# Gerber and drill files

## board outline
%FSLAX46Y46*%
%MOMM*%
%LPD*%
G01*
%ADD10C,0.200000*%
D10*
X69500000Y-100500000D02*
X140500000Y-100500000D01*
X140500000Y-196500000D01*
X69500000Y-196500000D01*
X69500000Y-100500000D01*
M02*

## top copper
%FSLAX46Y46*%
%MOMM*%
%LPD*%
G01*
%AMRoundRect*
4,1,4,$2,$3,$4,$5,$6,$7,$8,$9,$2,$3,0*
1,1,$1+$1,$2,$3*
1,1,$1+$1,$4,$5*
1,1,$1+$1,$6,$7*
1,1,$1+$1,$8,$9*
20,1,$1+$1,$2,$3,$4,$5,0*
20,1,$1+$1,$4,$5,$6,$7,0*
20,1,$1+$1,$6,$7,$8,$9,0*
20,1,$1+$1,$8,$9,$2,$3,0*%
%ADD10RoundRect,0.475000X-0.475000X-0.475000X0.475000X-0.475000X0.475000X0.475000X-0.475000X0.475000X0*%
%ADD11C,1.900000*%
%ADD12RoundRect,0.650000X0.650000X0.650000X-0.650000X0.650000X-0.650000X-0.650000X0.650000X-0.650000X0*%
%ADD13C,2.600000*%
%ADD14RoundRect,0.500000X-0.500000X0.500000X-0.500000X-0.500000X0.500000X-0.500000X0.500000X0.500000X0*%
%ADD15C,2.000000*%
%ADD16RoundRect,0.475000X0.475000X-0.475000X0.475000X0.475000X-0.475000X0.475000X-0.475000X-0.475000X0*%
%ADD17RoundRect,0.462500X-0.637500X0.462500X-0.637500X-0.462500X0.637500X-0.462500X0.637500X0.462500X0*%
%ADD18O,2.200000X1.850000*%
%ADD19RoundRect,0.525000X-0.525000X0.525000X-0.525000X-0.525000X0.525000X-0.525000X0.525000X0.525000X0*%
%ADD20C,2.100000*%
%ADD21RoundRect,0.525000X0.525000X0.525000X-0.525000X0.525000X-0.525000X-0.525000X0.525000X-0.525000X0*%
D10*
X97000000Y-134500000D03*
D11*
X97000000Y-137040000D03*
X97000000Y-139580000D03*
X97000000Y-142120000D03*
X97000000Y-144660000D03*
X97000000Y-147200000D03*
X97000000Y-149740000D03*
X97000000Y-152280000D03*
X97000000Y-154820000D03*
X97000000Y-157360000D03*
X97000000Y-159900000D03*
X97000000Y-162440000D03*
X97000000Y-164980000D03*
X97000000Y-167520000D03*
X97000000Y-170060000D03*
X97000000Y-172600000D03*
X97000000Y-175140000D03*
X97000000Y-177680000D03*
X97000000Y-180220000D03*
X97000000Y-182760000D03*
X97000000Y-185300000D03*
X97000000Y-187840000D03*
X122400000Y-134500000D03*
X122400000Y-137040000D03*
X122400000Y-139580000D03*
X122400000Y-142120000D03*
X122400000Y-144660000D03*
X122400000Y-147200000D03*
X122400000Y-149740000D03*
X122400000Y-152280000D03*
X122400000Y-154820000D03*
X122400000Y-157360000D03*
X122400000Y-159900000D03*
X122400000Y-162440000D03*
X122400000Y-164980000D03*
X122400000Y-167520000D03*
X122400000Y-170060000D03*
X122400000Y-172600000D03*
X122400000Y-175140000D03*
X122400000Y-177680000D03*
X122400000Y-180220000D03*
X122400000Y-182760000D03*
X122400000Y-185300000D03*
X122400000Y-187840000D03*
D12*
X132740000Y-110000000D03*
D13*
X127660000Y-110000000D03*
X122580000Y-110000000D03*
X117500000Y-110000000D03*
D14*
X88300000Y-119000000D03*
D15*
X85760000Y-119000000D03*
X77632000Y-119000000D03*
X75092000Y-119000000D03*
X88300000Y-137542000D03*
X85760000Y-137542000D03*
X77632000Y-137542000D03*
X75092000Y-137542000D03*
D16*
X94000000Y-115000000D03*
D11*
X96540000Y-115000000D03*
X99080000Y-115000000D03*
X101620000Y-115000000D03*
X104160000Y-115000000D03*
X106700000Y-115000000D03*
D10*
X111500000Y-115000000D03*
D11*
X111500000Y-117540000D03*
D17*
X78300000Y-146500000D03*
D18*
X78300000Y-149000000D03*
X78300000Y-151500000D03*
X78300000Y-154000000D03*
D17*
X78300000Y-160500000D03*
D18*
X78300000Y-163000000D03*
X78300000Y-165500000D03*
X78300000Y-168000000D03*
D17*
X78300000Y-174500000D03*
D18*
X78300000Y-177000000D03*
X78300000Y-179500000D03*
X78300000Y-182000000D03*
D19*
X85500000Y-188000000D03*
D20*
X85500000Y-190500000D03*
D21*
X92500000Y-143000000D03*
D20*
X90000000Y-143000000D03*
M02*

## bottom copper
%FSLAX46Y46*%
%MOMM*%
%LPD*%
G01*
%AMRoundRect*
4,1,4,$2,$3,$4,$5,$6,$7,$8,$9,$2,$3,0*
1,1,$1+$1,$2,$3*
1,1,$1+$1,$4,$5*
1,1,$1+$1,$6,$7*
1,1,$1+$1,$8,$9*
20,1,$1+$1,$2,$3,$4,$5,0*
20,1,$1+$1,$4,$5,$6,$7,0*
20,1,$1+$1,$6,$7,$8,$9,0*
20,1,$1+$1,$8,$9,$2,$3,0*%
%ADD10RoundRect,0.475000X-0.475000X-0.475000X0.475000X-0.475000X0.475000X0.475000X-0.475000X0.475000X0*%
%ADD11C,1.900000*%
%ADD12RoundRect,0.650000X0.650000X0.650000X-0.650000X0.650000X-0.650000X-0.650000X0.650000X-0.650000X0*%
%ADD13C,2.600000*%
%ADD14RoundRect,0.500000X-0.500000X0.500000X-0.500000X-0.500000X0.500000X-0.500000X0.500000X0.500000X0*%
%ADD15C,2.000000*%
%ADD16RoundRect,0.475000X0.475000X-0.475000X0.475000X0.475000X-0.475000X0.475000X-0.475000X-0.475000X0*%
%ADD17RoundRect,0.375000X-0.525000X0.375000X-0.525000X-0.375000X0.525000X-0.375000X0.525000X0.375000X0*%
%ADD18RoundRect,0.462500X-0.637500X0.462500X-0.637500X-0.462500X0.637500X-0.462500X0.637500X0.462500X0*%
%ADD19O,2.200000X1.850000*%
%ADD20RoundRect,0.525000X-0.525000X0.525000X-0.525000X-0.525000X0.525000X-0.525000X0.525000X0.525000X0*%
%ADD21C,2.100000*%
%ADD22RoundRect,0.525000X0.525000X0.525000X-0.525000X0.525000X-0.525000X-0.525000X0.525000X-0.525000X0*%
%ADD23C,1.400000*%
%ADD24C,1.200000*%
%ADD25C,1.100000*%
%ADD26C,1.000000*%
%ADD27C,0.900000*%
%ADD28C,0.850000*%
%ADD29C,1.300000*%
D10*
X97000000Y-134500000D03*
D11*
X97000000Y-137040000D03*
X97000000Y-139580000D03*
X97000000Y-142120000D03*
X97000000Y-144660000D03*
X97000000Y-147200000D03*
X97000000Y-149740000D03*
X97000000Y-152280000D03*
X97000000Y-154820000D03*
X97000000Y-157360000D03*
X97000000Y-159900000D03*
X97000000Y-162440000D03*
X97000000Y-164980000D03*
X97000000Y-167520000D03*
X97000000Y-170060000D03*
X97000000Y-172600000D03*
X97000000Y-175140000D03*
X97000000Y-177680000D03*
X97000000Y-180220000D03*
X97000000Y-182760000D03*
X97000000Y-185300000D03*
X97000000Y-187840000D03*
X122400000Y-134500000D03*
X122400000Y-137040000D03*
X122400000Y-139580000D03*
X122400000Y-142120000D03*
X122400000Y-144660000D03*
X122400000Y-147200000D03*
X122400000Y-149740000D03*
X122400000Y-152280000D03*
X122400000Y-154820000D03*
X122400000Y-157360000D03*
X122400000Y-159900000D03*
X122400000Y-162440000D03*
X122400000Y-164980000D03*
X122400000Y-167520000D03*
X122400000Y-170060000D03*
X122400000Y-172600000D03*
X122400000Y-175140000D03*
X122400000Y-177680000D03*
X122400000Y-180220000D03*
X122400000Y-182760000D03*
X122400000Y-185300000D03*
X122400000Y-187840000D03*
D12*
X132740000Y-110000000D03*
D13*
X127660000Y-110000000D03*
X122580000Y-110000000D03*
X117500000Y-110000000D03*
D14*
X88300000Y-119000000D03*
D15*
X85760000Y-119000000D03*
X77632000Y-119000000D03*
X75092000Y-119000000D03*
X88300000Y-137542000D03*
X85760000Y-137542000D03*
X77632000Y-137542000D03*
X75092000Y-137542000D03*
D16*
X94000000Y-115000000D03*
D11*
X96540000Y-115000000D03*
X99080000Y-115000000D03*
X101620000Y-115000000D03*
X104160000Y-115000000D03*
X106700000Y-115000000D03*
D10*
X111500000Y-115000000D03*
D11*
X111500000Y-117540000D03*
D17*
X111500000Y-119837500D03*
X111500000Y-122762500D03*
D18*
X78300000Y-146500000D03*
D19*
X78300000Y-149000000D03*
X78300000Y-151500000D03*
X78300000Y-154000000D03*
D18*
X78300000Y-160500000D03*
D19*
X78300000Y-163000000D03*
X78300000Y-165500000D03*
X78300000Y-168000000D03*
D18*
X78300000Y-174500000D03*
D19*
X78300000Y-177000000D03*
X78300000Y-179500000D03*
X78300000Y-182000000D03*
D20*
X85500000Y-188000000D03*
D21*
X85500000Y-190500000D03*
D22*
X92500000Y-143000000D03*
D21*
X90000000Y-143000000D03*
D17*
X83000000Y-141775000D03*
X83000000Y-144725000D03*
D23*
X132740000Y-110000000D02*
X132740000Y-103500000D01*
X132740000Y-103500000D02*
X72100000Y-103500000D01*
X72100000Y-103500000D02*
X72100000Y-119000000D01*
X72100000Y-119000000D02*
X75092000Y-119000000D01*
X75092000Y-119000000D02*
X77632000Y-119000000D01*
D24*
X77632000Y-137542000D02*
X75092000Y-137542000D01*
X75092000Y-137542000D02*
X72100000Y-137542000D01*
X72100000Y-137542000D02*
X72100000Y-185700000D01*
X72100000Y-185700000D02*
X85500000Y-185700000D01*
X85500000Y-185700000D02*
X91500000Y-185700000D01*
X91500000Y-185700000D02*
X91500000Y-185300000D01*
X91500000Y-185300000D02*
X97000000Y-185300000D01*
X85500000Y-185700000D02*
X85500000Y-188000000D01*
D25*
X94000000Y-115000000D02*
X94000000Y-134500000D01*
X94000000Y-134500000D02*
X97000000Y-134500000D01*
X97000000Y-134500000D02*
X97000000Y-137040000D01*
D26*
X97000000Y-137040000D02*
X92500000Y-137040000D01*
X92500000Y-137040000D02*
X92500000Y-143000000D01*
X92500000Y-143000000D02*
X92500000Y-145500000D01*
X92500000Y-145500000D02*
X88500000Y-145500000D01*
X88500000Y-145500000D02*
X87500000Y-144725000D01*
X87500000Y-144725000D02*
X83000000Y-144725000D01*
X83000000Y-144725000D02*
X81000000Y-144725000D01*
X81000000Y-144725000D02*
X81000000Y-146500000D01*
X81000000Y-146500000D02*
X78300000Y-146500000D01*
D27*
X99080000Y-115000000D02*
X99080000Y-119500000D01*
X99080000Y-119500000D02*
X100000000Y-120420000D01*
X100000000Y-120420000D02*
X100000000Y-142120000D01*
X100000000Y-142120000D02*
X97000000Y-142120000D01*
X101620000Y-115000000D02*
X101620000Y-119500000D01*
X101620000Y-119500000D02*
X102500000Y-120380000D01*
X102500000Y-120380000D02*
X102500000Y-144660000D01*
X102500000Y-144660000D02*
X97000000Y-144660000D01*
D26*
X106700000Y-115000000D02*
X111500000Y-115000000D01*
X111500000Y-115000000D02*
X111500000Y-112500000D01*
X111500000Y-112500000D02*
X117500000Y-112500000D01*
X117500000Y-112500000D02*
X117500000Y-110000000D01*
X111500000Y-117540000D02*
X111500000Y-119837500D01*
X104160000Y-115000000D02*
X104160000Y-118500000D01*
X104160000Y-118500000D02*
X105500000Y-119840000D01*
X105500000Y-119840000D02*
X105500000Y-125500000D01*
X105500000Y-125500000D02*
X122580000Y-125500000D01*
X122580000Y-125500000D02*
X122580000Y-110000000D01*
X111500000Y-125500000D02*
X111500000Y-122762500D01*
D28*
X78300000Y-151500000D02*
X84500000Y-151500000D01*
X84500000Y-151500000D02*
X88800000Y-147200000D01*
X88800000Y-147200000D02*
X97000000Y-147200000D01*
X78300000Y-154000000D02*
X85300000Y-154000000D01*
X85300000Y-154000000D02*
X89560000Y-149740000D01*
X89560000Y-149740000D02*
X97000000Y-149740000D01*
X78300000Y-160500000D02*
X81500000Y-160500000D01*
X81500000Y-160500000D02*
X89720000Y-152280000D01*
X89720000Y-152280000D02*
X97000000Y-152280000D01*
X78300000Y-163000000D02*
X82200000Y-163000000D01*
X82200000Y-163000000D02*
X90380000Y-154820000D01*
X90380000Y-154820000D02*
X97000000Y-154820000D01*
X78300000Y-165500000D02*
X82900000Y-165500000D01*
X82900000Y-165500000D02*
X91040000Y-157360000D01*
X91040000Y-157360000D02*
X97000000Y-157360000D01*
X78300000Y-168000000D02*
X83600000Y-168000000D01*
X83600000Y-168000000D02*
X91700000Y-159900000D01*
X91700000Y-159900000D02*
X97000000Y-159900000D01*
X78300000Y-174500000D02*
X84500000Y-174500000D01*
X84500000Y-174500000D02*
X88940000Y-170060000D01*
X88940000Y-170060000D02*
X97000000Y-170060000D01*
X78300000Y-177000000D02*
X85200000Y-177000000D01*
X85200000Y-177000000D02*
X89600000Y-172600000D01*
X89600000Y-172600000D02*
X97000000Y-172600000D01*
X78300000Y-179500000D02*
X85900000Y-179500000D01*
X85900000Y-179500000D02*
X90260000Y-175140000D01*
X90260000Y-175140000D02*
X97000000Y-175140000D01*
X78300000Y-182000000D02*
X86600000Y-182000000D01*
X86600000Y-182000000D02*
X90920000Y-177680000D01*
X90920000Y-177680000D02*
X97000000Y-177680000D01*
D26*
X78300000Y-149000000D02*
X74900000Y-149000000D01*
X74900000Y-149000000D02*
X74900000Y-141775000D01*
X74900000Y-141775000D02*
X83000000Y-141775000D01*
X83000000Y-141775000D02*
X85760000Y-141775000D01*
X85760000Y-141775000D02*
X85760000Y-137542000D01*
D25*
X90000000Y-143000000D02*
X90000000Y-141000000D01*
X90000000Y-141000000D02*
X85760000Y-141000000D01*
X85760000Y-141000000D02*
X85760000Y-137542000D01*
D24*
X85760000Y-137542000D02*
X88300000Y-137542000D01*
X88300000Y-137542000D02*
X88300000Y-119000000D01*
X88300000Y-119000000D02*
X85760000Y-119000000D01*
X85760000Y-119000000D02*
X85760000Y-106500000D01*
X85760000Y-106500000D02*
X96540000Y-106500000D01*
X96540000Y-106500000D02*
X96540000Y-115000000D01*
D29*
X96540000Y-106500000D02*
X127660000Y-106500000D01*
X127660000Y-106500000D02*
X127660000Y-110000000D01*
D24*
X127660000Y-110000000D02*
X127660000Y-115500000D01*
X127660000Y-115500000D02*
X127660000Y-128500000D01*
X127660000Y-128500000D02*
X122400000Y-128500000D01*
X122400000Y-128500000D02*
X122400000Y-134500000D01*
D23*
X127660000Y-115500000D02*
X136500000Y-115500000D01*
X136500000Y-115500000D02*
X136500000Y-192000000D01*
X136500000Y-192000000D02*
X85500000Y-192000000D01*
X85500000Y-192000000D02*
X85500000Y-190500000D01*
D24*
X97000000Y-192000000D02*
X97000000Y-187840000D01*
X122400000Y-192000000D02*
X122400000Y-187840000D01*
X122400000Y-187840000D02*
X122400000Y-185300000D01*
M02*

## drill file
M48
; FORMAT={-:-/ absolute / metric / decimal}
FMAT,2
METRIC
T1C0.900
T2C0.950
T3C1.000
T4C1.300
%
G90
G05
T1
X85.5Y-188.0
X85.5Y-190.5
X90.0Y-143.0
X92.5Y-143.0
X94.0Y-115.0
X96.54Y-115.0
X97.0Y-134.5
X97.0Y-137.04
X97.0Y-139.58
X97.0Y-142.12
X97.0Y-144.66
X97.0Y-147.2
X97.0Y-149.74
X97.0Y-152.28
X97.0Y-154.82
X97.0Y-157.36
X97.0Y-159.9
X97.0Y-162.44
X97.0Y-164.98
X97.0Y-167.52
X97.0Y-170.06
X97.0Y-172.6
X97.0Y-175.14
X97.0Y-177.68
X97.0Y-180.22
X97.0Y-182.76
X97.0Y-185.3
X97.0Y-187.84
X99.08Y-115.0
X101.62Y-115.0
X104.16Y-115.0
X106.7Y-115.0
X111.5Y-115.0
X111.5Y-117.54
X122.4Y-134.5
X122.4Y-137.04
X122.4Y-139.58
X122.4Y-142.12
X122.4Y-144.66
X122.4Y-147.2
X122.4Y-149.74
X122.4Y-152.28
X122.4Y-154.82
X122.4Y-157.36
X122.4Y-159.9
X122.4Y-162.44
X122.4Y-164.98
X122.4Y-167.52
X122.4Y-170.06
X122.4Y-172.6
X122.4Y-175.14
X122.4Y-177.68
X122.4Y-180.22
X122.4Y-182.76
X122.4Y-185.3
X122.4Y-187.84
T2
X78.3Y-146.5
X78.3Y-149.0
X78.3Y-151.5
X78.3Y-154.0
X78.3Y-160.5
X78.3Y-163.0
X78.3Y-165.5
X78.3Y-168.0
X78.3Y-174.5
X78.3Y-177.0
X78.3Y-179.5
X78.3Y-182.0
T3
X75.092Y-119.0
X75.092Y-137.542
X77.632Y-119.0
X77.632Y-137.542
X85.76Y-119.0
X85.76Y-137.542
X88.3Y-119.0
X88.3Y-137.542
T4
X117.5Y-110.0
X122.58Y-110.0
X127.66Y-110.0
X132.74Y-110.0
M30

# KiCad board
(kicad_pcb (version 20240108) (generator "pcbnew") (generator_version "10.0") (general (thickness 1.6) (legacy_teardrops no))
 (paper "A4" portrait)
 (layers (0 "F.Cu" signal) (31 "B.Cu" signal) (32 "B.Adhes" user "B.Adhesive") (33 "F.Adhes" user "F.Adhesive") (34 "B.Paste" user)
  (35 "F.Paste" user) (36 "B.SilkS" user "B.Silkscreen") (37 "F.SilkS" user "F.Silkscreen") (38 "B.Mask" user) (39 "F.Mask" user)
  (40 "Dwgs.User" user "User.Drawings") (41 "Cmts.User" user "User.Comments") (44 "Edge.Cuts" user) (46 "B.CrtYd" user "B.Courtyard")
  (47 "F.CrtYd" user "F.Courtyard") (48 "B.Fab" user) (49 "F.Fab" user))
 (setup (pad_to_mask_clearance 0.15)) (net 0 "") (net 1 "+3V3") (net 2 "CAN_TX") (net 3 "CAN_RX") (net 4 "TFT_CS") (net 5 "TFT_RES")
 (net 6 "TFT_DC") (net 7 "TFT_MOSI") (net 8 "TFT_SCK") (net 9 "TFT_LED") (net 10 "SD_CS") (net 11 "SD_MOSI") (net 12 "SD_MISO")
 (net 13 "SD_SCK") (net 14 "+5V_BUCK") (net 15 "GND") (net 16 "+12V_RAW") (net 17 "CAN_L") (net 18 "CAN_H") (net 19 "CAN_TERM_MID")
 (gr_rect (start 69.500 100.500) (end 140.500 196.500) (stroke (width 0.2) (type default)) (fill none) (layer "Edge.Cuts"))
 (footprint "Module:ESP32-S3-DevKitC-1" (layer "F.Cu") (at 97.0000 134.5000 0)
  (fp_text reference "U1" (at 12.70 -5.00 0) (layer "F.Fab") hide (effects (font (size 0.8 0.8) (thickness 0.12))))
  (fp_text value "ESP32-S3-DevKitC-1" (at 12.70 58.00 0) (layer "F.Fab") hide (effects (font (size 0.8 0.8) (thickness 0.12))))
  (pad "L1" thru_hole roundrect (at 0.0000 0.0000 0) (size 1.90 1.90) (drill 0.90) (layers "*.Cu" "*.Mask") (roundrect_rratio 0.25)
   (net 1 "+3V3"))
  (pad "L2" thru_hole circle (at 0.0000 2.5400 0) (size 1.90 1.90) (drill 0.90) (layers "*.Cu" "*.Mask") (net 1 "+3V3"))
  (pad "L3" thru_hole circle (at 0.0000 5.0800 0) (size 1.90 1.90) (drill 0.90) (layers "*.Cu" "*.Mask"))
  (pad "L4" thru_hole circle (at 0.0000 7.6200 0) (size 1.90 1.90) (drill 0.90) (layers "*.Cu" "*.Mask") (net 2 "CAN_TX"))
  (pad "L5" thru_hole circle (at 0.0000 10.1600 0) (size 1.90 1.90) (drill 0.90) (layers "*.Cu" "*.Mask") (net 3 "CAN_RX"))
  (pad "L6" thru_hole circle (at 0.0000 12.7000 0) (size 1.90 1.90) (drill 0.90) (layers "*.Cu" "*.Mask") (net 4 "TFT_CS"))
  (pad "L7" thru_hole circle (at 0.0000 15.2400 0) (size 1.90 1.90) (drill 0.90) (layers "*.Cu" "*.Mask") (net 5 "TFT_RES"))
  (pad "L8" thru_hole circle (at 0.0000 17.7800 0) (size 1.90 1.90) (drill 0.90) (layers "*.Cu" "*.Mask") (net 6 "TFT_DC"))
  (pad "L9" thru_hole circle (at 0.0000 20.3200 0) (size 1.90 1.90) (drill 0.90) (layers "*.Cu" "*.Mask") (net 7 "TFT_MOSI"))
  (pad "L10" thru_hole circle (at 0.0000 22.8600 0) (size 1.90 1.90) (drill 0.90) (layers "*.Cu" "*.Mask") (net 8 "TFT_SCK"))
  (pad "L11" thru_hole circle (at 0.0000 25.4000 0) (size 1.90 1.90) (drill 0.90) (layers "*.Cu" "*.Mask") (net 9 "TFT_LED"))
  (pad "L12" thru_hole circle (at 0.0000 27.9400 0) (size 1.90 1.90) (drill 0.90) (layers "*.Cu" "*.Mask"))
  (pad "L13" thru_hole circle (at 0.0000 30.4800 0) (size 1.90 1.90) (drill 0.90) (layers "*.Cu" "*.Mask"))
  (pad "L14" thru_hole circle (at 0.0000 33.0200 0) (size 1.90 1.90) (drill 0.90) (layers "*.Cu" "*.Mask"))
  (pad "L15" thru_hole circle (at 0.0000 35.5600 0) (size 1.90 1.90) (drill 0.90) (layers "*.Cu" "*.Mask") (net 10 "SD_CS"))
  (pad "L16" thru_hole circle (at 0.0000 38.1000 0) (size 1.90 1.90) (drill 0.90) (layers "*.Cu" "*.Mask") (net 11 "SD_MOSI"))
  (pad "L17" thru_hole circle (at 0.0000 40.6400 0) (size 1.90 1.90) (drill 0.90) (layers "*.Cu" "*.Mask") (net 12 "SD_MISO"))
  (pad "L18" thru_hole circle (at 0.0000 43.1800 0) (size 1.90 1.90) (drill 0.90) (layers "*.Cu" "*.Mask") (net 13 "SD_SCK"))
  (pad "L19" thru_hole circle (at 0.0000 45.7200 0) (size 1.90 1.90) (drill 0.90) (layers "*.Cu" "*.Mask"))
  (pad "L20" thru_hole circle (at 0.0000 48.2600 0) (size 1.90 1.90) (drill 0.90) (layers "*.Cu" "*.Mask"))
  (pad "L21" thru_hole circle (at 0.0000 50.8000 0) (size 1.90 1.90) (drill 0.90) (layers "*.Cu" "*.Mask") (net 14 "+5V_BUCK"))
  (pad "L22" thru_hole circle (at 0.0000 53.3400 0) (size 1.90 1.90) (drill 0.90) (layers "*.Cu" "*.Mask") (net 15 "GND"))
  (pad "R1" thru_hole circle (at 25.4000 0.0000 0) (size 1.90 1.90) (drill 0.90) (layers "*.Cu" "*.Mask") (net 15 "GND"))
  (pad "R2" thru_hole circle (at 25.4000 2.5400 0) (size 1.90 1.90) (drill 0.90) (layers "*.Cu" "*.Mask"))
  (pad "R3" thru_hole circle (at 25.4000 5.0800 0) (size 1.90 1.90) (drill 0.90) (layers "*.Cu" "*.Mask"))
  (pad "R4" thru_hole circle (at 25.4000 7.6200 0) (size 1.90 1.90) (drill 0.90) (layers "*.Cu" "*.Mask"))
  (pad "R5" thru_hole circle (at 25.4000 10.1600 0) (size 1.90 1.90) (drill 0.90) (layers "*.Cu" "*.Mask"))
  (pad "R6" thru_hole circle (at 25.4000 12.7000 0) (size 1.90 1.90) (drill 0.90) (layers "*.Cu" "*.Mask"))
  (pad "R7" thru_hole circle (at 25.4000 15.2400 0) (size 1.90 1.90) (drill 0.90) (layers "*.Cu" "*.Mask"))
  (pad "R8" thru_hole circle (at 25.4000 17.7800 0) (size 1.90 1.90) (drill 0.90) (layers "*.Cu" "*.Mask"))
  (pad "R9" thru_hole circle (at 25.4000 20.3200 0) (size 1.90 1.90) (drill 0.90) (layers "*.Cu" "*.Mask"))
  (pad "R10" thru_hole circle (at 25.4000 22.8600 0) (size 1.90 1.90) (drill 0.90) (layers "*.Cu" "*.Mask"))
  (pad "R11" thru_hole circle (at 25.4000 25.4000 0) (size 1.90 1.90) (drill 0.90) (layers "*.Cu" "*.Mask"))
  (pad "R12" thru_hole circle (at 25.4000 27.9400 0) (size 1.90 1.90) (drill 0.90) (layers "*.Cu" "*.Mask"))
  (pad "R13" thru_hole circle (at 25.4000 30.4800 0) (size 1.90 1.90) (drill 0.90) (layers "*.Cu" "*.Mask"))
  (pad "R14" thru_hole circle (at 25.4000 33.0200 0) (size 1.90 1.90) (drill 0.90) (layers "*.Cu" "*.Mask"))
  (pad "R15" thru_hole circle (at 25.4000 35.5600 0) (size 1.90 1.90) (drill 0.90) (layers "*.Cu" "*.Mask"))
  (pad "R16" thru_hole circle (at 25.4000 38.1000 0) (size 1.90 1.90) (drill 0.90) (layers "*.Cu" "*.Mask"))
  (pad "R17" thru_hole circle (at 25.4000 40.6400 0) (size 1.90 1.90) (drill 0.90) (layers "*.Cu" "*.Mask"))
  (pad "R18" thru_hole circle (at 25.4000 43.1800 0) (size 1.90 1.90) (drill 0.90) (layers "*.Cu" "*.Mask"))
  (pad "R19" thru_hole circle (at 25.4000 45.7200 0) (size 1.90 1.90) (drill 0.90) (layers "*.Cu" "*.Mask"))
  (pad "R20" thru_hole circle (at 25.4000 48.2600 0) (size 1.90 1.90) (drill 0.90) (layers "*.Cu" "*.Mask"))
  (pad "R21" thru_hole circle (at 25.4000 50.8000 0) (size 1.90 1.90) (drill 0.90) (layers "*.Cu" "*.Mask") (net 15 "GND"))
  (pad "R22" thru_hole circle (at 25.4000 53.3400 0) (size 1.90 1.90) (drill 0.90) (layers "*.Cu" "*.Mask") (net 15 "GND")))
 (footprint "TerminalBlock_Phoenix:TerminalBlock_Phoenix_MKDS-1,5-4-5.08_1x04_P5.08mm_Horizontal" (layer "F.Cu") (at 132.7400 110.0000 180)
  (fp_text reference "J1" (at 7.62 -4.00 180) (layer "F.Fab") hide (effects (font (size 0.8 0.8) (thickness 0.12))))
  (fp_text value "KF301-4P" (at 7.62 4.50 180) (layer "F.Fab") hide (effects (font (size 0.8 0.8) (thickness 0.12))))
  (pad "1" thru_hole roundrect (at 0.0000 0.0000 180) (size 2.60 2.60) (drill 1.30) (layers "*.Cu" "*.Mask") (roundrect_rratio 0.25)
   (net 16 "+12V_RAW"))
  (pad "2" thru_hole circle (at 5.0800 0.0000 180) (size 2.60 2.60) (drill 1.30) (layers "*.Cu" "*.Mask") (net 15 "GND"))
  (pad "3" thru_hole circle (at 10.1600 0.0000 180) (size 2.60 2.60) (drill 1.30) (layers "*.Cu" "*.Mask") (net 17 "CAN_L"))
  (pad "4" thru_hole circle (at 15.2400 0.0000 180) (size 2.60 2.60) (drill 1.30) (layers "*.Cu" "*.Mask") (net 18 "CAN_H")))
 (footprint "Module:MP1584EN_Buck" (layer "F.Cu") (at 88.3000 119.0000 270)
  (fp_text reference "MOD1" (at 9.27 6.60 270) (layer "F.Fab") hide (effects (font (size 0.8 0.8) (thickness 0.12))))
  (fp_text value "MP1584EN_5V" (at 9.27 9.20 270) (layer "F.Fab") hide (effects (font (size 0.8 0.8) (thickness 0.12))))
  (pad "1a" thru_hole roundrect (at 0.0000 0.0000 270) (size 2.00 2.00) (drill 1.00) (layers "*.Cu" "*.Mask") (roundrect_rratio 0.25)
   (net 15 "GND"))
  (pad "1b" thru_hole circle (at 0.0000 2.5400 270) (size 2.00 2.00) (drill 1.00) (layers "*.Cu" "*.Mask") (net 15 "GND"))
  (pad "2b" thru_hole circle (at 0.0000 10.6680 270) (size 2.00 2.00) (drill 1.00) (layers "*.Cu" "*.Mask") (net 16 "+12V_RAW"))
  (pad "2a" thru_hole circle (at 0.0000 13.2080 270) (size 2.00 2.00) (drill 1.00) (layers "*.Cu" "*.Mask") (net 16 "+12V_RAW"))
  (pad "3a" thru_hole circle (at 18.5420 0.0000 270) (size 2.00 2.00) (drill 1.00) (layers "*.Cu" "*.Mask") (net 15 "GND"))
  (pad "3b" thru_hole circle (at 18.5420 2.5400 270) (size 2.00 2.00) (drill 1.00) (layers "*.Cu" "*.Mask") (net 15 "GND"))
  (pad "4b" thru_hole circle (at 18.5420 10.6680 270) (size 2.00 2.00) (drill 1.00) (layers "*.Cu" "*.Mask") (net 14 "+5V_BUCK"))
  (pad "4a" thru_hole circle (at 18.5420 13.2080 270) (size 2.00 2.00) (drill 1.00) (layers "*.Cu" "*.Mask") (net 14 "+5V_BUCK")))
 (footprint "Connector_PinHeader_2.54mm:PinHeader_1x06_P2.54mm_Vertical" (layer "F.Cu") (at 94.0000 115.0000 90)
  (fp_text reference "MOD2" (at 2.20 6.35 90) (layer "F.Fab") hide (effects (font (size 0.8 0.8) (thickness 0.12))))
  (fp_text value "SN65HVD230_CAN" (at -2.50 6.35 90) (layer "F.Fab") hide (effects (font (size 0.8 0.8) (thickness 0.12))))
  (pad "1" thru_hole roundrect (at 0.0000 0.0000 90) (size 1.90 1.90) (drill 0.90) (layers "*.Cu" "*.Mask") (roundrect_rratio 0.25)
   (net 1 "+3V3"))
  (pad "2" thru_hole circle (at 0.0000 2.5400 90) (size 1.90 1.90) (drill 0.90) (layers "*.Cu" "*.Mask") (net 15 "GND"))
  (pad "3" thru_hole circle (at 0.0000 5.0800 90) (size 1.90 1.90) (drill 0.90) (layers "*.Cu" "*.Mask") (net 2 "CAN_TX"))
  (pad "4" thru_hole circle (at 0.0000 7.6200 90) (size 1.90 1.90) (drill 0.90) (layers "*.Cu" "*.Mask") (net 3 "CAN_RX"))
  (pad "5" thru_hole circle (at 0.0000 10.1600 90) (size 1.90 1.90) (drill 0.90) (layers "*.Cu" "*.Mask") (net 17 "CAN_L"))
  (pad "6" thru_hole circle (at 0.0000 12.7000 90) (size 1.90 1.90) (drill 0.90) (layers "*.Cu" "*.Mask") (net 18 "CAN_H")))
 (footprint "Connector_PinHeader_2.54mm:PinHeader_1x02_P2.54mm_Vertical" (layer "F.Cu") (at 111.5000 115.0000 0)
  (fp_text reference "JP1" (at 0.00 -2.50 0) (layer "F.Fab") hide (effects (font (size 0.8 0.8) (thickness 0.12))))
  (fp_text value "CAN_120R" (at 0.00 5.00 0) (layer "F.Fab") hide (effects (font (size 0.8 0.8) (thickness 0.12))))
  (pad "1" thru_hole roundrect (at 0.0000 0.0000 0) (size 1.90 1.90) (drill 0.90) (layers "*.Cu" "*.Mask") (roundrect_rratio 0.25)
   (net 18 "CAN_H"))
  (pad "2" thru_hole circle (at 0.0000 2.5400 0) (size 1.90 1.90) (drill 0.90) (layers "*.Cu" "*.Mask") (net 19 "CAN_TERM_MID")))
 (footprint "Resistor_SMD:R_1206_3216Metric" (layer "B.Cu") (at 111.5000 121.3000 270)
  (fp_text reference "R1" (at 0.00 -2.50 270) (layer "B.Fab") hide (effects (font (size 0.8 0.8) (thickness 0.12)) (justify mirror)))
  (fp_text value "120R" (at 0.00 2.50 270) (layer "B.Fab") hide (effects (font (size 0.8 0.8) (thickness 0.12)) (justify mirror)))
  (pad "1" smd roundrect (at -1.4625 0.0000 270) (size 1.50 1.80) (layers "B.Cu" "B.Mask" "B.Paste") (roundrect_rratio 0.25)
   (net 19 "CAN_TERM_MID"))
  (pad "2" smd roundrect (at 1.4625 0.0000 270) (size 1.50 1.80) (layers "B.Cu" "B.Mask" "B.Paste") (roundrect_rratio 0.25) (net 17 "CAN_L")))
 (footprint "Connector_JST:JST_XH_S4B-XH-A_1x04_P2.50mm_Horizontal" (layer "F.Cu") (at 78.3000 146.5000 270)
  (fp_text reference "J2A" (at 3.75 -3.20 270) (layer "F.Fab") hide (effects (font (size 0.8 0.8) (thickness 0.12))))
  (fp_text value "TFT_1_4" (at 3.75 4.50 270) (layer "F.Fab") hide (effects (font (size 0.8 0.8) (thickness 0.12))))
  (pad "1" thru_hole roundrect (at 0.0000 0.0000 270) (size 1.85 2.20) (drill 0.95) (layers "*.Cu" "*.Mask") (roundrect_rratio 0.25)
   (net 1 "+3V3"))
  (pad "2" thru_hole oval (at 2.5000 0.0000 270) (size 1.85 2.20) (drill 0.95) (layers "*.Cu" "*.Mask") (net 15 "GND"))
  (pad "3" thru_hole oval (at 5.0000 0.0000 270) (size 1.85 2.20) (drill 0.95) (layers "*.Cu" "*.Mask") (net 4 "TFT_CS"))
  (pad "4" thru_hole oval (at 7.5000 0.0000 270) (size 1.85 2.20) (drill 0.95) (layers "*.Cu" "*.Mask") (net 5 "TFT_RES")))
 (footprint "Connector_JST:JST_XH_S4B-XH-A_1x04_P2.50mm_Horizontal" (layer "F.Cu") (at 78.3000 160.5000 270)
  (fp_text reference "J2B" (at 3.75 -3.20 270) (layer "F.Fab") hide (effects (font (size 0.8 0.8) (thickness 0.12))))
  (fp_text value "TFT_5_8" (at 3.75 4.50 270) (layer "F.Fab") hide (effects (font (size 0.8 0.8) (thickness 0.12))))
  (pad "1" thru_hole roundrect (at 0.0000 0.0000 270) (size 1.85 2.20) (drill 0.95) (layers "*.Cu" "*.Mask") (roundrect_rratio 0.25)
   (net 6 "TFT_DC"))
  (pad "2" thru_hole oval (at 2.5000 0.0000 270) (size 1.85 2.20) (drill 0.95) (layers "*.Cu" "*.Mask") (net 7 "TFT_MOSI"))
  (pad "3" thru_hole oval (at 5.0000 0.0000 270) (size 1.85 2.20) (drill 0.95) (layers "*.Cu" "*.Mask") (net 8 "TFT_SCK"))
  (pad "4" thru_hole oval (at 7.5000 0.0000 270) (size 1.85 2.20) (drill 0.95) (layers "*.Cu" "*.Mask") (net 9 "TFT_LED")))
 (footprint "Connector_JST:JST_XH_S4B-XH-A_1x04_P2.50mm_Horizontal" (layer "F.Cu") (at 78.3000 174.5000 270)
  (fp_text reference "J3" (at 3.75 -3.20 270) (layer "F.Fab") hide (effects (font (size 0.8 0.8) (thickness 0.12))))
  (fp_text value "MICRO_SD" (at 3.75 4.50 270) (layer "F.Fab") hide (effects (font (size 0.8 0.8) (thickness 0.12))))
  (pad "1" thru_hole roundrect (at 0.0000 0.0000 270) (size 1.85 2.20) (drill 0.95) (layers "*.Cu" "*.Mask") (roundrect_rratio 0.25)
   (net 10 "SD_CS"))
  (pad "2" thru_hole oval (at 2.5000 0.0000 270) (size 1.85 2.20) (drill 0.95) (layers "*.Cu" "*.Mask") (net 11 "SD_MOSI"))
  (pad "3" thru_hole oval (at 5.0000 0.0000 270) (size 1.85 2.20) (drill 0.95) (layers "*.Cu" "*.Mask") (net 12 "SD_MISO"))
  (pad "4" thru_hole oval (at 7.5000 0.0000 270) (size 1.85 2.20) (drill 0.95) (layers "*.Cu" "*.Mask") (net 13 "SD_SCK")))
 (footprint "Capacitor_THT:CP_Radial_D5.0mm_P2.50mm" (layer "F.Cu") (at 85.5000 188.0000 270)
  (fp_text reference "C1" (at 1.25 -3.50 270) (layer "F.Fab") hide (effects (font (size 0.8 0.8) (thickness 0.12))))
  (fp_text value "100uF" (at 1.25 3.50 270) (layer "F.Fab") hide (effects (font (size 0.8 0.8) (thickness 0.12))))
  (pad "1" thru_hole roundrect (at 0.0000 0.0000 270) (size 2.10 2.10) (drill 0.90) (layers "*.Cu" "*.Mask") (roundrect_rratio 0.25)
   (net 14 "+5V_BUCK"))
  (pad "2" thru_hole circle (at 2.5000 0.0000 270) (size 2.10 2.10) (drill 0.90) (layers "*.Cu" "*.Mask") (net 15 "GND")))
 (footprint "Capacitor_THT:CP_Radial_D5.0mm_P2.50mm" (layer "F.Cu") (at 92.5000 143.0000 180)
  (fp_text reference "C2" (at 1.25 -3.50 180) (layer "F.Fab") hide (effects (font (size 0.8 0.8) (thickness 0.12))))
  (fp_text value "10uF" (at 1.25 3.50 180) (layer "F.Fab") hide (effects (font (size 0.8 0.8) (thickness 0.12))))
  (pad "1" thru_hole roundrect (at 0.0000 0.0000 180) (size 2.10 2.10) (drill 0.90) (layers "*.Cu" "*.Mask") (roundrect_rratio 0.25)
   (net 1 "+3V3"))
  (pad "2" thru_hole circle (at 2.5000 0.0000 180) (size 2.10 2.10) (drill 0.90) (layers "*.Cu" "*.Mask") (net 15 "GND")))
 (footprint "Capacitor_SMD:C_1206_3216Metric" (layer "B.Cu") (at 83.0000 143.2500 270)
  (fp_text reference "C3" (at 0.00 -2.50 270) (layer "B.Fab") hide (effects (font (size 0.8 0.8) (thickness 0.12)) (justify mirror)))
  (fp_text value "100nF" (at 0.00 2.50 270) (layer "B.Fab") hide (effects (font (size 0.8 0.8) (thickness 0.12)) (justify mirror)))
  (pad "1" smd roundrect (at -1.4750 0.0000 270) (size 1.50 1.80) (layers "B.Cu" "B.Mask" "B.Paste") (roundrect_rratio 0.25) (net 15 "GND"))
  (pad "2" smd roundrect (at 1.4750 0.0000 270) (size 1.50 1.80) (layers "B.Cu" "B.Mask" "B.Paste") (roundrect_rratio 0.25) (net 1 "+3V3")))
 (segment (start 132.7400 110.0000) (end 132.7400 103.5000) (width 1.40) (layer "B.Cu") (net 16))
 (segment (start 132.7400 103.5000) (end 72.1000 103.5000) (width 1.40) (layer "B.Cu") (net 16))
 (segment (start 72.1000 103.5000) (end 72.1000 119.0000) (width 1.40) (layer "B.Cu") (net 16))
 (segment (start 72.1000 119.0000) (end 75.0920 119.0000) (width 1.40) (layer "B.Cu") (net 16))
 (segment (start 75.0920 119.0000) (end 77.6320 119.0000) (width 1.40) (layer "B.Cu") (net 16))
 (segment (start 77.6320 137.5420) (end 75.0920 137.5420) (width 1.20) (layer "B.Cu") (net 14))
 (segment (start 75.0920 137.5420) (end 72.1000 137.5420) (width 1.20) (layer "B.Cu") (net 14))
 (segment (start 72.1000 137.5420) (end 72.1000 185.7000) (width 1.20) (layer "B.Cu") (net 14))
 (segment (start 72.1000 185.7000) (end 85.5000 185.7000) (width 1.20) (layer "B.Cu") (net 14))
 (segment (start 85.5000 185.7000) (end 91.5000 185.7000) (width 1.20) (layer "B.Cu") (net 14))
 (segment (start 91.5000 185.7000) (end 91.5000 185.3000) (width 1.20) (layer "B.Cu") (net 14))
 (segment (start 91.5000 185.3000) (end 97.0000 185.3000) (width 1.20) (layer "B.Cu") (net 14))
 (segment (start 85.5000 185.7000) (end 85.5000 188.0000) (width 1.20) (layer "B.Cu") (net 14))
 (segment (start 94.0000 115.0000) (end 94.0000 134.5000) (width 1.10) (layer "B.Cu") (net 1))
 (segment (start 94.0000 134.5000) (end 97.0000 134.5000) (width 1.10) (layer "B.Cu") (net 1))
 (segment (start 97.0000 134.5000) (end 97.0000 137.0400) (width 1.10) (layer "B.Cu") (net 1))
 (segment (start 97.0000 137.0400) (end 92.5000 137.0400) (width 1.00) (layer "B.Cu") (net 1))
 (segment (start 92.5000 137.0400) (end 92.5000 143.0000) (width 1.00) (layer "B.Cu") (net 1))
 (segment (start 92.5000 143.0000) (end 92.5000 145.5000) (width 1.00) (layer "B.Cu") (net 1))
 (segment (start 92.5000 145.5000) (end 88.5000 145.5000) (width 1.00) (layer "B.Cu") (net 1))
 (segment (start 88.5000 145.5000) (end 87.5000 144.7250) (width 1.00) (layer "B.Cu") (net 1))
 (segment (start 87.5000 144.7250) (end 83.0000 144.7250) (width 1.00) (layer "B.Cu") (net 1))
 (segment (start 83.0000 144.7250) (end 81.0000 144.7250) (width 1.00) (layer "B.Cu") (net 1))
 (segment (start 81.0000 144.7250) (end 81.0000 146.5000) (width 1.00) (layer "B.Cu") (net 1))
 (segment (start 81.0000 146.5000) (end 78.3000 146.5000) (width 1.00) (layer "B.Cu") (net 1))
 (segment (start 99.0800 115.0000) (end 99.0800 119.5000) (width 0.90) (layer "B.Cu") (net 2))
 (segment (start 99.0800 119.5000) (end 100.0000 120.4200) (width 0.90) (layer "B.Cu") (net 2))
 (segment (start 100.0000 120.4200) (end 100.0000 142.1200) (width 0.90) (layer "B.Cu") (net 2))
 (segment (start 100.0000 142.1200) (end 97.0000 142.1200) (width 0.90) (layer "B.Cu") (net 2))
 (segment (start 101.6200 115.0000) (end 101.6200 119.5000) (width 0.90) (layer "B.Cu") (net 3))
 (segment (start 101.6200 119.5000) (end 102.5000 120.3800) (width 0.90) (layer "B.Cu") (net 3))
 (segment (start 102.5000 120.3800) (end 102.5000 144.6600) (width 0.90) (layer "B.Cu") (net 3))
 (segment (start 102.5000 144.6600) (end 97.0000 144.6600) (width 0.90) (layer "B.Cu") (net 3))
 (segment (start 106.7000 115.0000) (end 111.5000 115.0000) (width 1.00) (layer "B.Cu") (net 18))
 (segment (start 111.5000 115.0000) (end 111.5000 112.5000) (width 1.00) (layer "B.Cu") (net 18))
 (segment (start 111.5000 112.5000) (end 117.5000 112.5000) (width 1.00) (layer "B.Cu") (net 18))
 (segment (start 117.5000 112.5000) (end 117.5000 110.0000) (width 1.00) (layer "B.Cu") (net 18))
 (segment (start 111.5000 117.5400) (end 111.5000 119.8375) (width 1.00) (layer "B.Cu") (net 19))
 (segment (start 104.1600 115.0000) (end 104.1600 118.5000) (width 1.00) (layer "B.Cu") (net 17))
 (segment (start 104.1600 118.5000) (end 105.5000 119.8400) (width 1.00) (layer "B.Cu") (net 17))
 (segment (start 105.5000 119.8400) (end 105.5000 125.5000) (width 1.00) (layer "B.Cu") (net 17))
 (segment (start 105.5000 125.5000) (end 122.5800 125.5000) (width 1.00) (layer "B.Cu") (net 17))
 (segment (start 122.5800 125.5000) (end 122.5800 110.0000) (width 1.00) (layer "B.Cu") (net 17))
 (segment (start 111.5000 125.5000) (end 111.5000 122.7625) (width 1.00) (layer "B.Cu") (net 17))
 (segment (start 78.3000 151.5000) (end 84.5000 151.5000) (width 0.85) (layer "B.Cu") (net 4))
 (segment (start 84.5000 151.5000) (end 88.8000 147.2000) (width 0.85) (layer "B.Cu") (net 4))
 (segment (start 88.8000 147.2000) (end 97.0000 147.2000) (width 0.85) (layer "B.Cu") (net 4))
 (segment (start 78.3000 154.0000) (end 85.3000 154.0000) (width 0.85) (layer "B.Cu") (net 5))
 (segment (start 85.3000 154.0000) (end 89.5600 149.7400) (width 0.85) (layer "B.Cu") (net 5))
 (segment (start 89.5600 149.7400) (end 97.0000 149.7400) (width 0.85) (layer "B.Cu") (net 5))
 (segment (start 78.3000 160.5000) (end 81.5000 160.5000) (width 0.85) (layer "B.Cu") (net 6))
 (segment (start 81.5000 160.5000) (end 89.7200 152.2800) (width 0.85) (layer "B.Cu") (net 6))
 (segment (start 89.7200 152.2800) (end 97.0000 152.2800) (width 0.85) (layer "B.Cu") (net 6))
 (segment (start 78.3000 163.0000) (end 82.2000 163.0000) (width 0.85) (layer "B.Cu") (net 7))
 (segment (start 82.2000 163.0000) (end 90.3800 154.8200) (width 0.85) (layer "B.Cu") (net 7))
 (segment (start 90.3800 154.8200) (end 97.0000 154.8200) (width 0.85) (layer "B.Cu") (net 7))
 (segment (start 78.3000 165.5000) (end 82.9000 165.5000) (width 0.85) (layer "B.Cu") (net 8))
 (segment (start 82.9000 165.5000) (end 91.0400 157.3600) (width 0.85) (layer "B.Cu") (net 8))
 (segment (start 91.0400 157.3600) (end 97.0000 157.3600) (width 0.85) (layer "B.Cu") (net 8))
 (segment (start 78.3000 168.0000) (end 83.6000 168.0000) (width 0.85) (layer "B.Cu") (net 9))
 (segment (start 83.6000 168.0000) (end 91.7000 159.9000) (width 0.85) (layer "B.Cu") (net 9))
 (segment (start 91.7000 159.9000) (end 97.0000 159.9000) (width 0.85) (layer "B.Cu") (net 9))
 (segment (start 78.3000 174.5000) (end 84.5000 174.5000) (width 0.85) (layer "B.Cu") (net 10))
 (segment (start 84.5000 174.5000) (end 88.9400 170.0600) (width 0.85) (layer "B.Cu") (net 10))
 (segment (start 88.9400 170.0600) (end 97.0000 170.0600) (width 0.85) (layer "B.Cu") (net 10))
 (segment (start 78.3000 177.0000) (end 85.2000 177.0000) (width 0.85) (layer "B.Cu") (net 11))
 (segment (start 85.2000 177.0000) (end 89.6000 172.6000) (width 0.85) (layer "B.Cu") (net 11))
 (segment (start 89.6000 172.6000) (end 97.0000 172.6000) (width 0.85) (layer "B.Cu") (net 11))
 (segment (start 78.3000 179.5000) (end 85.9000 179.5000) (width 0.85) (layer "B.Cu") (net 12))
 (segment (start 85.9000 179.5000) (end 90.2600 175.1400) (width 0.85) (layer "B.Cu") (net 12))
 (segment (start 90.2600 175.1400) (end 97.0000 175.1400) (width 0.85) (layer "B.Cu") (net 12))
 (segment (start 78.3000 182.0000) (end 86.6000 182.0000) (width 0.85) (layer "B.Cu") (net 13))
 (segment (start 86.6000 182.0000) (end 90.9200 177.6800) (width 0.85) (layer "B.Cu") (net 13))
 (segment (start 90.9200 177.6800) (end 97.0000 177.6800) (width 0.85) (layer "B.Cu") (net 13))
 (segment (start 78.3000 149.0000) (end 74.9000 149.0000) (width 1.00) (layer "B.Cu") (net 15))
 (segment (start 74.9000 149.0000) (end 74.9000 141.7750) (width 1.00) (layer "B.Cu") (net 15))
 (segment (start 74.9000 141.7750) (end 83.0000 141.7750) (width 1.00) (layer "B.Cu") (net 15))
 (segment (start 83.0000 141.7750) (end 85.7600 141.7750) (width 1.00) (layer "B.Cu") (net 15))
 (segment (start 85.7600 141.7750) (end 85.7600 137.5420) (width 1.00) (layer "B.Cu") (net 15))
 (segment (start 90.0000 143.0000) (end 90.0000 141.0000) (width 1.10) (layer "B.Cu") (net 15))
 (segment (start 90.0000 141.0000) (end 85.7600 141.0000) (width 1.10) (layer "B.Cu") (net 15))
 (segment (start 85.7600 141.0000) (end 85.7600 137.5420) (width 1.10) (layer "B.Cu") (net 15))
 (segment (start 85.7600 137.5420) (end 88.3000 137.5420) (width 1.20) (layer "B.Cu") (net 15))
 (segment (start 88.3000 137.5420) (end 88.3000 119.0000) (width 1.20) (layer "B.Cu") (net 15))
 (segment (start 88.3000 119.0000) (end 85.7600 119.0000) (width 1.20) (layer "B.Cu") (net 15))
 (segment (start 85.7600 119.0000) (end 85.7600 106.5000) (width 1.20) (layer "B.Cu") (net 15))
 (segment (start 85.7600 106.5000) (end 96.5400 106.5000) (width 1.20) (layer "B.Cu") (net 15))
 (segment (start 96.5400 106.5000) (end 96.5400 115.0000) (width 1.20) (layer "B.Cu") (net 15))
 (segment (start 96.5400 106.5000) (end 127.6600 106.5000) (width 1.30) (layer "B.Cu") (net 15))
 (segment (start 127.6600 106.5000) (end 127.6600 110.0000) (width 1.30) (layer "B.Cu") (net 15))
 (segment (start 127.6600 110.0000) (end 127.6600 115.5000) (width 1.20) (layer "B.Cu") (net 15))
 (segment (start 127.6600 115.5000) (end 127.6600 128.5000) (width 1.20) (layer "B.Cu") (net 15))
 (segment (start 127.6600 128.5000) (end 122.4000 128.5000) (width 1.20) (layer "B.Cu") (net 15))
 (segment (start 122.4000 128.5000) (end 122.4000 134.5000) (width 1.20) (layer "B.Cu") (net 15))
 (segment (start 127.6600 115.5000) (end 136.5000 115.5000) (width 1.40) (layer "B.Cu") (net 15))
 (segment (start 136.5000 115.5000) (end 136.5000 192.0000) (width 1.40) (layer "B.Cu") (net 15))
 (segment (start 136.5000 192.0000) (end 85.5000 192.0000) (width 1.40) (layer "B.Cu") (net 15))
 (segment (start 85.5000 192.0000) (end 85.5000 190.5000) (width 1.40) (layer "B.Cu") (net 15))
 (segment (start 97.0000 192.0000) (end 97.0000 187.8400) (width 1.20) (layer "B.Cu") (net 15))
 (segment (start 122.4000 192.0000) (end 122.4000 187.8400) (width 1.20) (layer "B.Cu") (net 15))
 (segment (start 122.4000 187.8400) (end 122.4000 185.3000) (width 1.20) (layer "B.Cu") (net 15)))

